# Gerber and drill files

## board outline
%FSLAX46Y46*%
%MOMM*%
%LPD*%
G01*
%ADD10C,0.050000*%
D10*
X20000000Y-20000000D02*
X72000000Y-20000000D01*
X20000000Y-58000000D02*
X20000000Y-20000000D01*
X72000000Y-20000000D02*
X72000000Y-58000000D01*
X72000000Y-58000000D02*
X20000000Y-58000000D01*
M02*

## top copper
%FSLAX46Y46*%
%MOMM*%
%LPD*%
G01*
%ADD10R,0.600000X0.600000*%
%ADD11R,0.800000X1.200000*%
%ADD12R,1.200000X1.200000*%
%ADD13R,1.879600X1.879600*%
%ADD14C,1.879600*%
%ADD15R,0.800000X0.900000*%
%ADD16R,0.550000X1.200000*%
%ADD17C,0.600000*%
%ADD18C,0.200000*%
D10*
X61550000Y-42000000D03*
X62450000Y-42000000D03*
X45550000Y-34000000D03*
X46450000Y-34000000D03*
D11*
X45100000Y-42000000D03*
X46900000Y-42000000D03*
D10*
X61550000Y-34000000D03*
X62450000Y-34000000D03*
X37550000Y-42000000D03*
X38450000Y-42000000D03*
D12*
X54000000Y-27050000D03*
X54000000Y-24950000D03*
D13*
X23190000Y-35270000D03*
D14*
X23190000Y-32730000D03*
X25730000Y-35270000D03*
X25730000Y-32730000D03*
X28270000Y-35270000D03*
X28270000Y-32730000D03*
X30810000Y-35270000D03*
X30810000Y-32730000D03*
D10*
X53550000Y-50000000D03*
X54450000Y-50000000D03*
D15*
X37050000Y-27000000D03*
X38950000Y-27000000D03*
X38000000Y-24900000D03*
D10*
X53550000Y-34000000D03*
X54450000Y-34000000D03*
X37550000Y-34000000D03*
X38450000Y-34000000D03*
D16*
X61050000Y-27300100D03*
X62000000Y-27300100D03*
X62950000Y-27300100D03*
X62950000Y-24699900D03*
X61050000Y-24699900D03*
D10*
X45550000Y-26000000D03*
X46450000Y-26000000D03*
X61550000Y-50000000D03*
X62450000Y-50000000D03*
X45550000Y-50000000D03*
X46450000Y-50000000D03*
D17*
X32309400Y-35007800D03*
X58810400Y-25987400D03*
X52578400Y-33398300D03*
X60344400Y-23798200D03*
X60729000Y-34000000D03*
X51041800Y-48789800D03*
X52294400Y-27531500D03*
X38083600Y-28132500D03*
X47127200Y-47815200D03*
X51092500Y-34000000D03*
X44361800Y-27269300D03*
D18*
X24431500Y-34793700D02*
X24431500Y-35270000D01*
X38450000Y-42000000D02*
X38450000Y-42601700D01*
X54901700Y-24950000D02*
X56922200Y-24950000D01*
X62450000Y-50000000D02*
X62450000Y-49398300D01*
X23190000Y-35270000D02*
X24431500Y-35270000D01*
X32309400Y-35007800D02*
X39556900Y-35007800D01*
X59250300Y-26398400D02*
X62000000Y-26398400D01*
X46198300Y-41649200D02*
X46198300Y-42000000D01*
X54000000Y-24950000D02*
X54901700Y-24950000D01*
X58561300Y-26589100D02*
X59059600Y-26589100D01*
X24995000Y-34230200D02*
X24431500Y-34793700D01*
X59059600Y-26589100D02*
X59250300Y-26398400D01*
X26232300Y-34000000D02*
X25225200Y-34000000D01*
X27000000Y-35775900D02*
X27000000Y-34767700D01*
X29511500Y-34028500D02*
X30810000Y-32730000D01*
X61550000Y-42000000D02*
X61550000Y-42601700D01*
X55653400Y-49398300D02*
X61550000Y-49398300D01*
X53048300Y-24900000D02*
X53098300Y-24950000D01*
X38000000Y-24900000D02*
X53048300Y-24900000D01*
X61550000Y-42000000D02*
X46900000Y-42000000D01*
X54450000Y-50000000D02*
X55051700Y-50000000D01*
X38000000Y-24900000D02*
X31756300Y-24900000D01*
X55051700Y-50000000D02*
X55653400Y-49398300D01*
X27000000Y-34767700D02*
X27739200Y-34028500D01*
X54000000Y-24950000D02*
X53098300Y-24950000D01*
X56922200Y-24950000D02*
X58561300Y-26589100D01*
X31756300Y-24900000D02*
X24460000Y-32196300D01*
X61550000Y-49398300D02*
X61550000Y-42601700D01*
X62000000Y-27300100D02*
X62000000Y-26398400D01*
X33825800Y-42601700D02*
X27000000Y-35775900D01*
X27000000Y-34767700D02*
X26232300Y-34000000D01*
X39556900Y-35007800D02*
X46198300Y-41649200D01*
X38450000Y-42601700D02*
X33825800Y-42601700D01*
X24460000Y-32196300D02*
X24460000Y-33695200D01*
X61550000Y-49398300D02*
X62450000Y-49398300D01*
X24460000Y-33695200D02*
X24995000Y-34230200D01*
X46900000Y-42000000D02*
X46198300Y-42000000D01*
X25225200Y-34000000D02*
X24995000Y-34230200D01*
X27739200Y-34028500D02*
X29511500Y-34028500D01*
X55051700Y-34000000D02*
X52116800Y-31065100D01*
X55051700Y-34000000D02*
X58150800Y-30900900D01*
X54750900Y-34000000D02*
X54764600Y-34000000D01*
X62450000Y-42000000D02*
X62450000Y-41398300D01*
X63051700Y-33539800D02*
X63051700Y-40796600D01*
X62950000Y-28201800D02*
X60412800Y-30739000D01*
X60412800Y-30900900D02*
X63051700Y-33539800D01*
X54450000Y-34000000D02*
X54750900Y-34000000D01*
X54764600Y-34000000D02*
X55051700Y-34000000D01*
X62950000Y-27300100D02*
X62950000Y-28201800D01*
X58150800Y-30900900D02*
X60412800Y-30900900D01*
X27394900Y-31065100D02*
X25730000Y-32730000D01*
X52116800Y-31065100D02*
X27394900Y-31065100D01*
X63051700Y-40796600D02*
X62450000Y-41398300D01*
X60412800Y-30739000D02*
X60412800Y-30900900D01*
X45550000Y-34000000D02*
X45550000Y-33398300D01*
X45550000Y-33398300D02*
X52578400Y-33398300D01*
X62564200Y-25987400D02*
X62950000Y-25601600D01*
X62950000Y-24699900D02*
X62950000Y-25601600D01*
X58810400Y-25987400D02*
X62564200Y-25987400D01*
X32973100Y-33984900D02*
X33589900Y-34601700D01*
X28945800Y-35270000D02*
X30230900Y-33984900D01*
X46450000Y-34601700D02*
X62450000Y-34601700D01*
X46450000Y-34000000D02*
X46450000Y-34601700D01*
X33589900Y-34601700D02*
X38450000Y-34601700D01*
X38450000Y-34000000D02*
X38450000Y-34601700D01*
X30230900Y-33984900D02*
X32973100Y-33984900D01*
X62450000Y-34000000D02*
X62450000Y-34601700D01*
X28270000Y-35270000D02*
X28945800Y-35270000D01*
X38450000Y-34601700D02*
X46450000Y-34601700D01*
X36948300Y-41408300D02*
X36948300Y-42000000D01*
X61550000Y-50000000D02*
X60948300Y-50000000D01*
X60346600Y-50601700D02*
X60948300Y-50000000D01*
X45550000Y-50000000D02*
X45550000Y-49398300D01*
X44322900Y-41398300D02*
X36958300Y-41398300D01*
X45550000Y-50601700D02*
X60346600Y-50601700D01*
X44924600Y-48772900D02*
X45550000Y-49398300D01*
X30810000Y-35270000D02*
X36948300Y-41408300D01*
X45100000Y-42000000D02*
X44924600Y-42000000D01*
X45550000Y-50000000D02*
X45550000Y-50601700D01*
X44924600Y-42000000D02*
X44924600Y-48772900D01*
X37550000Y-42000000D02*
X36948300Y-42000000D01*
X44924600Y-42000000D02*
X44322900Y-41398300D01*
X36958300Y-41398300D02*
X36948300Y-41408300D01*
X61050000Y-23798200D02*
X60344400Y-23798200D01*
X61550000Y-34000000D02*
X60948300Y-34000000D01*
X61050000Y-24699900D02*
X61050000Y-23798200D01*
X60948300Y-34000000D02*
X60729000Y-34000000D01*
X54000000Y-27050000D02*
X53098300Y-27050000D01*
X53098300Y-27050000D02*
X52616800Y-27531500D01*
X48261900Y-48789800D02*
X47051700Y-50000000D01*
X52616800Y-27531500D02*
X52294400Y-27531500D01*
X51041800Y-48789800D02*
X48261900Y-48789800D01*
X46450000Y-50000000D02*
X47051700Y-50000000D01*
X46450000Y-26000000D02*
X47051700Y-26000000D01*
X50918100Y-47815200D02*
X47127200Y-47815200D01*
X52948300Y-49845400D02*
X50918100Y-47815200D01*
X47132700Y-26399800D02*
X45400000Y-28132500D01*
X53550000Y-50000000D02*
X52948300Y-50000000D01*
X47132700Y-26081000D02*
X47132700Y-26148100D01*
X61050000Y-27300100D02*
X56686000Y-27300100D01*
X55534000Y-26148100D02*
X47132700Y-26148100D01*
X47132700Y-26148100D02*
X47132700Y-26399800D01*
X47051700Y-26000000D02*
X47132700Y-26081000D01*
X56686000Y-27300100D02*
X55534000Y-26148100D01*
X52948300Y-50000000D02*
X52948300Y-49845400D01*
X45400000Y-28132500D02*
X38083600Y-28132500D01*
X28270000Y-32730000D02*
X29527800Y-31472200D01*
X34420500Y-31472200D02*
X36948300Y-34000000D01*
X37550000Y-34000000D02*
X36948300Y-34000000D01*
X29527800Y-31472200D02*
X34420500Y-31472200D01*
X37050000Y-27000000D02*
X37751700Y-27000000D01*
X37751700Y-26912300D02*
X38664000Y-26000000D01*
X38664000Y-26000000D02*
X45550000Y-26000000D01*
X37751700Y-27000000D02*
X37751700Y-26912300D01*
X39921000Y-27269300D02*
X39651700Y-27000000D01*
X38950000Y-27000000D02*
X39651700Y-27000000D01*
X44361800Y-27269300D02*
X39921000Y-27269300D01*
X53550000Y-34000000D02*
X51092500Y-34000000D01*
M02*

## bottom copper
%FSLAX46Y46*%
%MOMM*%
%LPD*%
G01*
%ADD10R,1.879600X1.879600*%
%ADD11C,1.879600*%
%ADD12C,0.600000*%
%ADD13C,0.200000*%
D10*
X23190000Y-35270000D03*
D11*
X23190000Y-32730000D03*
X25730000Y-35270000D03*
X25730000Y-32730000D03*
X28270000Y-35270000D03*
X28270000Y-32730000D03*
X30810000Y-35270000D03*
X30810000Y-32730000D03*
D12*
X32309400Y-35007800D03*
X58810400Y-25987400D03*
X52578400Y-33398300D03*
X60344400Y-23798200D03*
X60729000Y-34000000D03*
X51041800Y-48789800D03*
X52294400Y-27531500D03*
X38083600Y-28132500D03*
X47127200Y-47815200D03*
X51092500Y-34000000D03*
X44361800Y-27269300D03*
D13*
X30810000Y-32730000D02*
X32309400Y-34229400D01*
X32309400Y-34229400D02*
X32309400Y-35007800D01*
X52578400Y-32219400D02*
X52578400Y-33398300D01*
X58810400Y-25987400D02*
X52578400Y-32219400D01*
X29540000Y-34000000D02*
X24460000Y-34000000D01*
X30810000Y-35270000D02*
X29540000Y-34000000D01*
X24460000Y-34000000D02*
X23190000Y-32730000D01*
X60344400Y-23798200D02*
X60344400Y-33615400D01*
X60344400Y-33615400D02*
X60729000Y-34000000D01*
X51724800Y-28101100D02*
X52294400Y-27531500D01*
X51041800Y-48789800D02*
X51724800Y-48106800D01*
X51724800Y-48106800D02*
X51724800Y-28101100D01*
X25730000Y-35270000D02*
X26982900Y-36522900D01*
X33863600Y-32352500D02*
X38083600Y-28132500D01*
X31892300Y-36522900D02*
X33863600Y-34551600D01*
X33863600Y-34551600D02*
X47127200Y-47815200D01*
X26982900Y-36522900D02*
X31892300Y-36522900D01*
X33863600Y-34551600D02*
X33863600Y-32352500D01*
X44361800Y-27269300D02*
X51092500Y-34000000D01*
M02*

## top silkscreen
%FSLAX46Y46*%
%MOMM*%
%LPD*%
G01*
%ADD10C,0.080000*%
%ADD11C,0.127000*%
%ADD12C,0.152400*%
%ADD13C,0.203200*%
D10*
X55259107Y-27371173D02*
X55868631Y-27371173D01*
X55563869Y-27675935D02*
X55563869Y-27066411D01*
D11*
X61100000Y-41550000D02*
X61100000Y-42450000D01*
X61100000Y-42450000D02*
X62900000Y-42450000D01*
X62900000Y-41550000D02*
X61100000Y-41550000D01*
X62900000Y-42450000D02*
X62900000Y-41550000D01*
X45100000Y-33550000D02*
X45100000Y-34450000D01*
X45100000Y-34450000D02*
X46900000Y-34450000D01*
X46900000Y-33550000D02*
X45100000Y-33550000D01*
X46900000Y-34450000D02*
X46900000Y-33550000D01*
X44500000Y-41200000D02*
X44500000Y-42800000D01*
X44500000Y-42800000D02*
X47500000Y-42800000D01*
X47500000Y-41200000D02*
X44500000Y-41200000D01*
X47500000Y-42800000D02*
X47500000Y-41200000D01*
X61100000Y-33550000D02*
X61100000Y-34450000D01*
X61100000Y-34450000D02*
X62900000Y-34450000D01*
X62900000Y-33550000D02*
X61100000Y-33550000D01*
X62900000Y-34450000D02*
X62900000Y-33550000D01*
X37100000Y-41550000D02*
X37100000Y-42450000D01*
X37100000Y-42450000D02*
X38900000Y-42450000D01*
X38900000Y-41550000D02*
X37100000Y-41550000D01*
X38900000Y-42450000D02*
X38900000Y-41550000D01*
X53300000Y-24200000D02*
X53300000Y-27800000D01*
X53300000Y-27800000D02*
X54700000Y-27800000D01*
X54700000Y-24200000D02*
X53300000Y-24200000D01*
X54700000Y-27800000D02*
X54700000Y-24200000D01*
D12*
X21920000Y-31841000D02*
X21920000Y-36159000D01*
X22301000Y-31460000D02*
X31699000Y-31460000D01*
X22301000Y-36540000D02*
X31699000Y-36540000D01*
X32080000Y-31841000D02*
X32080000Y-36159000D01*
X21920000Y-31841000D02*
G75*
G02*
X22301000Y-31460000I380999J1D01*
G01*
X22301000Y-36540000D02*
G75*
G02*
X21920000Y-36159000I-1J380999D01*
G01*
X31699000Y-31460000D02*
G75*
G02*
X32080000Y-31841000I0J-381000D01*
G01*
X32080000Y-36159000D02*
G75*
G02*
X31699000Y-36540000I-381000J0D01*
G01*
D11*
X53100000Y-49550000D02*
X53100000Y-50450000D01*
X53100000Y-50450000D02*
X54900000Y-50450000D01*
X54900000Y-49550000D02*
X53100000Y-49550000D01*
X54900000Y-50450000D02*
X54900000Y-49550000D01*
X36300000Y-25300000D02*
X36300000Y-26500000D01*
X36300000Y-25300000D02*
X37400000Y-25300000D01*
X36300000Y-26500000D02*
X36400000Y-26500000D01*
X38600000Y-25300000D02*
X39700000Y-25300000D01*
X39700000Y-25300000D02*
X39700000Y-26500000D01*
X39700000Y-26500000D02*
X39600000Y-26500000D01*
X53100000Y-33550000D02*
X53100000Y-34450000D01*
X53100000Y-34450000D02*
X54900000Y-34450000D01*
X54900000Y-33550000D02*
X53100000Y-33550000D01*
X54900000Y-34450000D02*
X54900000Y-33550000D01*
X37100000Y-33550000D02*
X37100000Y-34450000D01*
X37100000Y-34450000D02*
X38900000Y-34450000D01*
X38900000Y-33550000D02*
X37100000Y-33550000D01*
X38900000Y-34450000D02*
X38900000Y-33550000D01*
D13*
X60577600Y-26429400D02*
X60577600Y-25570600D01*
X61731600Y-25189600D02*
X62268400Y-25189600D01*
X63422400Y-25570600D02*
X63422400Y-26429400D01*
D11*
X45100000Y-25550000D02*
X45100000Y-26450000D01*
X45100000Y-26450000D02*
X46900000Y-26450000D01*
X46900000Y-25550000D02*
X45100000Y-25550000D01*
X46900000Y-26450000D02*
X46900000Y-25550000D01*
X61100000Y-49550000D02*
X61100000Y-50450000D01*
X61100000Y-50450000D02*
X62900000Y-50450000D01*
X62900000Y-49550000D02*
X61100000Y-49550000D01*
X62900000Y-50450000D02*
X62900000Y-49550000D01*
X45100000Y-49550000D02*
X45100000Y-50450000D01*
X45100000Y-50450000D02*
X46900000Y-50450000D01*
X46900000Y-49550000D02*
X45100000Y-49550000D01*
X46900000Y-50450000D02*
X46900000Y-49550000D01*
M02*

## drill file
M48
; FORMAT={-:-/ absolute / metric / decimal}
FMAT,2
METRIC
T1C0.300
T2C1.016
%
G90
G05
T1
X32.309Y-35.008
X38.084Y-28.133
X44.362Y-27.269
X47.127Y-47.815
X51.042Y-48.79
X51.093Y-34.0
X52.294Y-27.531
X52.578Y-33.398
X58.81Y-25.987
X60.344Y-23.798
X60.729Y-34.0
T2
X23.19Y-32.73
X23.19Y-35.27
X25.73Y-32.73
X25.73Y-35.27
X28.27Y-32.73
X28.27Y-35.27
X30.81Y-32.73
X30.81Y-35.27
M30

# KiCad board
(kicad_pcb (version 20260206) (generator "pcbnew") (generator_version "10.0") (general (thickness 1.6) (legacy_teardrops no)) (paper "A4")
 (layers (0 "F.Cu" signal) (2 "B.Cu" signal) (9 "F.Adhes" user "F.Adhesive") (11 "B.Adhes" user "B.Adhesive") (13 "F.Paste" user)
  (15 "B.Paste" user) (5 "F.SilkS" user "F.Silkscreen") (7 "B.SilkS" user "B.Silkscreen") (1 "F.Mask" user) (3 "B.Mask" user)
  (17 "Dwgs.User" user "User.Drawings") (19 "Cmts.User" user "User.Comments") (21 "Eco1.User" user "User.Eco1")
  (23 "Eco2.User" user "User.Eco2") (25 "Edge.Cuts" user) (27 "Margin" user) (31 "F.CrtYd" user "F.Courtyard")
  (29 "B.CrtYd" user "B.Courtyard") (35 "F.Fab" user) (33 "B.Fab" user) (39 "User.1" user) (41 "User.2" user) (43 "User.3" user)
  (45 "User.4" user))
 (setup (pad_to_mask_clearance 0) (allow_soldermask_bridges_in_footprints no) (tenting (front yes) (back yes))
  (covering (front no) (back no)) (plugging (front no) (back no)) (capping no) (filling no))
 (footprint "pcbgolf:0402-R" (layer "F.Cu") (at 62 42)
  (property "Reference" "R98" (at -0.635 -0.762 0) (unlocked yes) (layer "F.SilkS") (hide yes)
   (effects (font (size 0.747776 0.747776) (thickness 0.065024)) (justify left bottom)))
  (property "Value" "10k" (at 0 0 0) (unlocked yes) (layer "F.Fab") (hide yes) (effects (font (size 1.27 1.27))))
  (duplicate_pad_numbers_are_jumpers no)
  (fp_line (start -0.9 -0.45) (end -0.9 0.45) (stroke (width 0.127) (type solid)) (layer "F.SilkS"))
  (fp_line (start -0.9 0.45) (end 0.9 0.45) (stroke (width 0.127) (type solid)) (layer "F.SilkS"))
  (fp_line (start 0.9 -0.45) (end -0.9 -0.45) (stroke (width 0.127) (type solid)) (layer "F.SilkS"))
  (fp_line (start 0.9 0.45) (end 0.9 -0.45) (stroke (width 0.127) (type solid)) (layer "F.SilkS"))
  (pad "1" smd rect (at -0.45 0) (size 0.6 0.6) (layers "F.Cu" "F.Mask" "F.Paste") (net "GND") (solder_mask_margin 0.0508)
   (solder_paste_margin 0) (thermal_bridge_angle 0))
  (pad "2" smd rect (at 0.45 0) (size 0.6 0.6) (layers "F.Cu" "F.Mask" "F.Paste") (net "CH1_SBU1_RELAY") (solder_mask_margin 0.0508)
   (solder_paste_margin 0) (thermal_bridge_angle 0)))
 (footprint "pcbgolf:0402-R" (layer "F.Cu") (at 46 34)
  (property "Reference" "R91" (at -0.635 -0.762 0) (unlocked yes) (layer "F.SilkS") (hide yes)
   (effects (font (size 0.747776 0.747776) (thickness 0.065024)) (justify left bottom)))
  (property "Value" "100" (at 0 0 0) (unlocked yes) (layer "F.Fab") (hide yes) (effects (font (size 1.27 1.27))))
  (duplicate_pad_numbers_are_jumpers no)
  (fp_line (start -0.9 -0.45) (end -0.9 0.45) (stroke (width 0.127) (type solid)) (layer "F.SilkS"))
  (fp_line (start -0.9 0.45) (end 0.9 0.45) (stroke (width 0.127) (type solid)) (layer "F.SilkS"))
  (fp_line (start 0.9 -0.45) (end -0.9 -0.45) (stroke (width 0.127) (type solid)) (layer "F.SilkS"))
  (fp_line (start 0.9 0.45) (end 0.9 -0.45) (stroke (width 0.127) (type solid)) (layer "F.SilkS"))
  (pad "1" smd rect (at -0.45 0) (size 0.6 0.6) (layers "F.Cu" "F.Mask" "F.Paste") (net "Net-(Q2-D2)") (solder_mask_margin 0.0508)
   (solder_paste_margin 0) (thermal_bridge_angle 0))
  (pad "2" smd rect (at 0.45 0) (size 0.6 0.6) (layers "F.Cu" "F.Mask" "F.Paste") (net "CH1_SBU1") (solder_mask_margin 0.0508)
   (solder_paste_margin 0) (thermal_bridge_angle 0)))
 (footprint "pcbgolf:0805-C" (layer "F.Cu") (at 46 42)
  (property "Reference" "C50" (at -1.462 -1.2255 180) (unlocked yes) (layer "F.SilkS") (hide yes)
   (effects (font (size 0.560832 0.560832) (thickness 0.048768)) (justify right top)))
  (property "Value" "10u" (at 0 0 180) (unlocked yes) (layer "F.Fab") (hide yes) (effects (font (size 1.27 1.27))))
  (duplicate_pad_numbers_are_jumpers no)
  (fp_line (start -1.5 -0.8) (end -1.5 0.8) (stroke (width 0.127) (type solid)) (layer "F.SilkS"))
  (fp_line (start -1.5 0.8) (end 1.5 0.8) (stroke (width 0.127) (type solid)) (layer "F.SilkS"))
  (fp_line (start 1.5 -0.8) (end -1.5 -0.8) (stroke (width 0.127) (type solid)) (layer "F.SilkS"))
  (fp_line (start 1.5 0.8) (end 1.5 -0.8) (stroke (width 0.127) (type solid)) (layer "F.SilkS"))
  (pad "1" smd rect (at -0.9 0) (size 0.8 1.2) (layers "F.Cu" "F.Mask" "F.Paste") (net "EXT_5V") (solder_mask_margin 0.0508)
   (solder_paste_margin 0) (thermal_bridge_angle 0))
  (pad "2" smd rect (at 0.9 0) (size 0.8 1.2) (layers "F.Cu" "F.Mask" "F.Paste") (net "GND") (solder_mask_margin 0.0508)
   (solder_paste_margin 0) (thermal_bridge_angle 0)))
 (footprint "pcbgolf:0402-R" (layer "F.Cu") (at 62 34)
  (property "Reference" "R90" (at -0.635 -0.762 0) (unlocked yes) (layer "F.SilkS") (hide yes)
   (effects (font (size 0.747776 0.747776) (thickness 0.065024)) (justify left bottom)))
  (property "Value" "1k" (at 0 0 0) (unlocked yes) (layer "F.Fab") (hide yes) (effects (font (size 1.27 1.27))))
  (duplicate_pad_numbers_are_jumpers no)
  (fp_line (start -0.9 -0.45) (end -0.9 0.45) (stroke (width 0.127) (type solid)) (layer "F.SilkS"))
  (fp_line (start -0.9 0.45) (end 0.9 0.45) (stroke (width 0.127) (type solid)) (layer "F.SilkS"))
  (fp_line (start 0.9 -0.45) (end -0.9 -0.45) (stroke (width 0.127) (type solid)) (layer "F.SilkS"))
  (fp_line (start 0.9 0.45) (end 0.9 -0.45) (stroke (width 0.127) (type solid)) (layer "F.SilkS"))
  (pad "1" smd rect (at -0.45 0) (size 0.6 0.6) (layers "F.Cu" "F.Mask" "F.Paste") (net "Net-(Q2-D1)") (solder_mask_margin 0.0508)
   (solder_paste_margin 0) (thermal_bridge_angle 0))
  (pad "2" smd rect (at 0.45 0) (size 0.6 0.6) (layers "F.Cu" "F.Mask" "F.Paste") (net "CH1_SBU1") (solder_mask_margin 0.0508)
   (solder_paste_margin 0) (thermal_bridge_angle 0)))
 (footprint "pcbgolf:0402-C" (layer "F.Cu") (at 38 42)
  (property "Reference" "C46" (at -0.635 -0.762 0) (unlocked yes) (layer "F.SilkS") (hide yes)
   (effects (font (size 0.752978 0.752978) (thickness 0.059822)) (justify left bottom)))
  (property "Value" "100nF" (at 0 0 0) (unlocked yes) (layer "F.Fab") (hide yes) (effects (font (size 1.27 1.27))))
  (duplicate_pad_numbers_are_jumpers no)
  (fp_line (start -0.9 -0.45) (end -0.9 0.45) (stroke (width 0.127) (type solid)) (layer "F.SilkS"))
  (fp_line (start -0.9 0.45) (end 0.9 0.45) (stroke (width 0.127) (type solid)) (layer "F.SilkS"))
  (fp_line (start 0.9 -0.45) (end -0.9 -0.45) (stroke (width 0.127) (type solid)) (layer "F.SilkS"))
  (fp_line (start 0.9 0.45) (end 0.9 -0.45) (stroke (width 0.127) (type solid)) (layer "F.SilkS"))
  (pad "1" smd rect (at -0.45 0) (size 0.6 0.6) (layers "F.Cu" "F.Mask" "F.Paste") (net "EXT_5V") (solder_mask_margin 0.0508)
   (solder_paste_margin 0) (thermal_bridge_angle 0))
  (pad "2" smd rect (at 0.45 0) (size 0.6 0.6) (layers "F.Cu" "F.Mask" "F.Paste") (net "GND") (solder_mask_margin 0.0508)
   (solder_paste_margin 0) (thermal_bridge_angle 0)))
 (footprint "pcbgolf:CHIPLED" (layer "F.Cu") (at 54 26)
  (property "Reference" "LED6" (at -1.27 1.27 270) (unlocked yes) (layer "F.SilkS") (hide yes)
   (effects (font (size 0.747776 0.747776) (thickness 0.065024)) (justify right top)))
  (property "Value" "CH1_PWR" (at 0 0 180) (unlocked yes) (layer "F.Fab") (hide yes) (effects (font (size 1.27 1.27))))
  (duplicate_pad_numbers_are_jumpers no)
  (fp_line (start -0.7 -1.8) (end -0.7 1.8) (stroke (width 0.127) (type solid)) (layer "F.SilkS"))
  (fp_line (start -0.7 1.8) (end 0.7 1.8) (stroke (width 0.127) (type solid)) (layer "F.SilkS"))
  (fp_line (start 0.7 -1.8) (end -0.7 -1.8) (stroke (width 0.127) (type solid)) (layer "F.SilkS"))
  (fp_line (start 0.7 1.8) (end 0.7 -1.8) (stroke (width 0.127) (type solid)) (layer "F.SilkS"))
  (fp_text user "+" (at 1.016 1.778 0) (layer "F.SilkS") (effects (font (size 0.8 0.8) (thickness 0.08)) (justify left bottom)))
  (pad "A" smd rect (at 0 1.05) (size 1.2 1.2) (layers "F.Cu" "F.Mask" "F.Paste") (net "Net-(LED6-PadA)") (solder_mask_margin 0.0508)
   (solder_paste_margin 0) (thermal_bridge_angle 0))
  (pad "C" smd rect (at 0 -1.05) (size 1.2 1.2) (layers "F.Cu" "F.Mask" "F.Paste") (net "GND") (solder_mask_margin 0.0508)
   (solder_paste_margin 0) (thermal_bridge_angle 0)))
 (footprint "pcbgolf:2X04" (layer "F.Cu") (at 27 34)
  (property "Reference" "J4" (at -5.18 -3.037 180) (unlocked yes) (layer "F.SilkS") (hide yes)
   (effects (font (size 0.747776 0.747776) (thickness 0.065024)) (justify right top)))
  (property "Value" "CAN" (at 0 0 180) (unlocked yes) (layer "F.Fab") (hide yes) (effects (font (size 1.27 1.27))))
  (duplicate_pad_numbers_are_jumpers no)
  (fp_line (start -5.08 -2.159) (end -5.08 2.159) (stroke (width 0.1524) (type solid)) (layer "F.SilkS"))
  (fp_line (start -4.699 -2.54) (end 4.699 -2.54) (stroke (width 0.1524) (type solid)) (layer "F.SilkS"))
  (fp_line (start -4.699 2.54) (end 4.699 2.54) (stroke (width 0.1524) (type solid)) (layer "F.SilkS"))
  (fp_line (start 5.08 -2.159) (end 5.08 2.159) (stroke (width 0.1524) (type solid)) (layer "F.SilkS"))
  (fp_arc (start -5.08 -2.159) (mid -4.968408 -2.428408) (end -4.699 -2.54) (stroke (width 0.1524) (type solid)) (layer "F.SilkS"))
  (fp_arc (start -4.699 2.54) (mid -4.968408 2.428408) (end -5.08 2.159) (stroke (width 0.1524) (type solid)) (layer "F.SilkS"))
  (fp_arc (start 4.699 -2.54) (mid 4.968408 -2.428408) (end 5.08 -2.159) (stroke (width 0.1524) (type solid)) (layer "F.SilkS"))
  (fp_arc (start 5.08 2.159) (mid 4.968408 2.428408) (end 4.699 2.54) (stroke (width 0.1524) (type solid)) (layer "F.SilkS"))
  (pad "1" thru_hole rect (at -3.81 1.27 90) (size 1.8796 1.8796) (drill 1.016) (layers "*.Cu" "*.Mask") (remove_unused_layers no)
   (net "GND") (solder_mask_margin 0.0508) (thermal_bridge_angle 0))
  (pad "2" thru_hole circle (at -3.81 -1.27 90) (size 1.8796 1.8796) (drill 1.016) (layers "*.Cu" "*.Mask") (remove_unused_layers no)
   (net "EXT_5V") (solder_mask_margin 0.0508) (thermal_bridge_angle 0))
  (pad "3" thru_hole circle (at -1.27 1.27 90) (size 1.8796 1.8796) (drill 1.016) (layers "*.Cu" "*.Mask") (remove_unused_layers no)
   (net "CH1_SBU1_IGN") (solder_mask_margin 0.0508) (thermal_bridge_angle 0))
  (pad "4" thru_hole circle (at -1.27 -1.27 90) (size 1.8796 1.8796) (drill 1.016) (layers "*.Cu" "*.Mask") (remove_unused_layers no)
   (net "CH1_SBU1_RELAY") (solder_mask_margin 0.0508) (thermal_bridge_angle 0))
  (pad "5" thru_hole circle (at 1.27 1.27 90) (size 1.8796 1.8796) (drill 1.016) (layers "*.Cu" "*.Mask") (remove_unused_layers no)
   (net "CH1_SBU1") (solder_mask_margin 0.0508) (thermal_bridge_angle 0))
  (pad "6" thru_hole circle (at 1.27 -1.27 90) (size 1.8796 1.8796) (drill 1.016) (layers "*.Cu" "*.Mask") (remove_unused_layers no)
   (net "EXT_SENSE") (solder_mask_margin 0.0508) (thermal_bridge_angle 0))
  (pad "7" thru_hole circle (at 3.81 1.27 90) (size 1.8796 1.8796) (drill 1.016) (layers "*.Cu" "*.Mask") (remove_unused_layers no)
   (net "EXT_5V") (solder_mask_margin 0.0508) (thermal_bridge_angle 0))
  (pad "8" thru_hole circle (at 3.81 -1.27 90) (size 1.8796 1.8796) (drill 1.016) (layers "*.Cu" "*.Mask") (remove_unused_layers no)
   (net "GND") (solder_mask_margin 0.0508) (thermal_bridge_angle 0)))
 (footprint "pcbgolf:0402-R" (layer "F.Cu") (at 54 50)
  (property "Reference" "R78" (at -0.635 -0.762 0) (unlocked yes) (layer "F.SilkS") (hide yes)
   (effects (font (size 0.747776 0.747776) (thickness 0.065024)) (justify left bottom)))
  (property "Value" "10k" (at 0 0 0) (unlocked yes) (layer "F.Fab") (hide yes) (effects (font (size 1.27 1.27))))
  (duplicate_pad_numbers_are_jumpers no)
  (fp_line (start -0.9 -0.45) (end -0.9 0.45) (stroke (width 0.127) (type solid)) (layer "F.SilkS"))
  (fp_line (start -0.9 0.45) (end 0.9 0.45) (stroke (width 0.127) (type solid)) (layer "F.SilkS"))
  (fp_line (start 0.9 -0.45) (end -0.9 -0.45) (stroke (width 0.127) (type solid)) (layer "F.SilkS"))
  (fp_line (start 0.9 0.45) (end 0.9 -0.45) (stroke (width 0.127) (type solid)) (layer "F.SilkS"))
  (pad "1" smd rect (at -0.45 0) (size 0.6 0.6) (layers "F.Cu" "F.Mask" "F.Paste") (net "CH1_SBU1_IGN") (solder_mask_margin 0.0508)
   (solder_paste_margin 0) (thermal_bridge_angle 0))
  (pad "2" smd rect (at 0.45 0) (size 0.6 0.6) (layers "F.Cu" "F.Mask" "F.Paste") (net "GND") (solder_mask_margin 0.0508)
   (solder_paste_margin 0) (thermal_bridge_angle 0)))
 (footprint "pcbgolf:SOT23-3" (layer "F.Cu") (at 38 26)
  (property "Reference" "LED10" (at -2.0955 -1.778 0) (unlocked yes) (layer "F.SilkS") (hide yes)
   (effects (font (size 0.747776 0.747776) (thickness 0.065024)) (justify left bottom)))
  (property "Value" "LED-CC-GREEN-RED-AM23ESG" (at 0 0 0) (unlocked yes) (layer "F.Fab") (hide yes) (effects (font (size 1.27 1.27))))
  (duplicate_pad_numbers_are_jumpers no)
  (fp_line (start -1.7 -0.7) (end -1.7 0.5) (stroke (width 0.127) (type solid)) (layer "F.SilkS"))
  (fp_line (start -1.7 -0.7) (end -0.6 -0.7) (stroke (width 0.127) (type solid)) (layer "F.SilkS"))
  (fp_line (start -1.7 0.5) (end -1.6 0.5) (stroke (width 0.127) (type solid)) (layer "F.SilkS"))
  (fp_line (start 0.6 -0.7) (end 1.7 -0.7) (stroke (width 0.127) (type solid)) (layer "F.SilkS"))
  (fp_line (start 1.7 -0.7) (end 1.7 0.5) (stroke (width 0.127) (type solid)) (layer "F.SilkS"))
  (fp_line (start 1.7 0.5) (end 1.6 0.5) (stroke (width 0.127) (type solid)) (layer "F.SilkS"))
  (pad "1" smd rect (at -0.95 1) (size 0.8 0.9) (layers "F.Cu" "F.Mask" "F.Paste") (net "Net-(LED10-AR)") (solder_mask_margin 0.0508)
   (solder_paste_margin 0) (thermal_bridge_angle 0))
  (pad "2" smd rect (at 0.95 1) (size 0.8 0.9) (layers "F.Cu" "F.Mask" "F.Paste") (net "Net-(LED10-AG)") (solder_mask_margin 0.0508)
   (solder_paste_margin 0) (thermal_bridge_angle 0))
  (pad "3" smd rect (at 0 -1.1) (size 0.8 0.9) (layers "F.Cu" "F.Mask" "F.Paste") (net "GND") (solder_mask_margin 0.0508)
   (solder_paste_margin 0) (thermal_bridge_angle 0)))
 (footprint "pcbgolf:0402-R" (layer "F.Cu") (at 54 34)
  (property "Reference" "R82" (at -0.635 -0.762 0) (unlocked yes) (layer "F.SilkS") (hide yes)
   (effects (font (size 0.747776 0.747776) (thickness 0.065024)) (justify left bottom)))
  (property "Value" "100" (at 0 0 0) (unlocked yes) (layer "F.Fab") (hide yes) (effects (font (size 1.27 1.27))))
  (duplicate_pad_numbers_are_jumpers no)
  (fp_line (start -0.9 -0.45) (end -0.9 0.45) (stroke (width 0.127) (type solid)) (layer "F.SilkS"))
  (fp_line (start -0.9 0.45) (end 0.9 0.45) (stroke (width 0.127) (type solid)) (layer "F.SilkS"))
  (fp_line (start 0.9 -0.45) (end -0.9 -0.45) (stroke (width 0.127) (type solid)) (layer "F.SilkS"))
  (fp_line (start 0.9 0.45) (end 0.9 -0.45) (stroke (width 0.127) (type solid)) (layer "F.SilkS"))
  (pad "1" smd rect (at -0.45 0) (size 0.6 0.6) (layers "F.Cu" "F.Mask" "F.Paste") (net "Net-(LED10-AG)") (solder_mask_margin 0.0508)
   (solder_paste_margin 0) (thermal_bridge_angle 0))
  (pad "2" smd rect (at 0.45 0) (size 0.6 0.6) (layers "F.Cu" "F.Mask" "F.Paste") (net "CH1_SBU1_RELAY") (solder_mask_margin 0.0508)
   (solder_paste_margin 0) (thermal_bridge_angle 0)))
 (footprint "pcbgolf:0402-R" (layer "F.Cu") (at 38 34)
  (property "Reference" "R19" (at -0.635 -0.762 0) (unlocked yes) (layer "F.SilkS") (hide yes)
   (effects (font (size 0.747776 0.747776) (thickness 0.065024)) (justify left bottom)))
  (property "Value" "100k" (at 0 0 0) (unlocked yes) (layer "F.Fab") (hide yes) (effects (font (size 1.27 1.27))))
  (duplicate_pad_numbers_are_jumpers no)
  (fp_line (start -0.9 -0.45) (end -0.9 0.45) (stroke (width 0.127) (type solid)) (layer "F.SilkS"))
  (fp_line (start -0.9 0.45) (end 0.9 0.45) (stroke (width 0.127) (type solid)) (layer "F.SilkS"))
  (fp_line (start 0.9 -0.45) (end -0.9 -0.45) (stroke (width 0.127) (type solid)) (layer "F.SilkS"))
  (fp_line (start 0.9 0.45) (end 0.9 -0.45) (stroke (width 0.127) (type solid)) (layer "F.SilkS"))
  (pad "1" smd rect (at -0.45 0) (size 0.6 0.6) (layers "F.Cu" "F.Mask" "F.Paste") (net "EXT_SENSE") (solder_mask_margin 0.0508)
   (solder_paste_margin 0) (thermal_bridge_angle 0))
  (pad "2" smd rect (at 0.45 0) (size 0.6 0.6) (layers "F.Cu" "F.Mask" "F.Paste") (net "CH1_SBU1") (solder_mask_margin 0.0508)
   (solder_paste_margin 0) (thermal_bridge_angle 0)))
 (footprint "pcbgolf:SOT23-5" (layer "F.Cu") (at 62 26)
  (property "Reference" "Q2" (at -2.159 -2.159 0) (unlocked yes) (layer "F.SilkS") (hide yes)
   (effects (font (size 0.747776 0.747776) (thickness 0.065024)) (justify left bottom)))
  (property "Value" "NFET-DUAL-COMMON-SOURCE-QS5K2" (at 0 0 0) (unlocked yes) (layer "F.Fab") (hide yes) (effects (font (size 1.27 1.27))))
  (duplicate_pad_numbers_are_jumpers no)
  (fp_line (start -1.4224 0.4294) (end -1.4224 -0.4294) (stroke (width 0.2032) (type solid)) (layer "F.SilkS"))
  (fp_line (start -0.2684 -0.8104) (end 0.2684 -0.8104) (stroke (width 0.2032) (type solid)) (layer "F.SilkS"))
  (fp_line (start 1.4224 -0.4294) (end 1.4224 0.4294) (stroke (width 0.2032) (type solid)) (layer "F.SilkS"))
  (pad "1" smd rect (at -0.95 1.3001) (size 0.55 1.2) (layers "F.Cu" "F.Mask" "F.Paste") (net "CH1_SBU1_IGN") (solder_mask_margin 0.0508)
   (solder_paste_margin 0) (thermal_bridge_angle 0))
  (pad "2" smd rect (at 0 1.3001) (size 0.55 1.2) (layers "F.Cu" "F.Mask" "F.Paste") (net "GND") (solder_mask_margin 0.0508)
   (solder_paste_margin 0) (thermal_bridge_angle 0))
  (pad "3" smd rect (at 0.95 1.3001) (size 0.55 1.2) (layers "F.Cu" "F.Mask" "F.Paste") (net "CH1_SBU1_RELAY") (solder_mask_margin 0.0508)
   (solder_paste_margin 0) (thermal_bridge_angle 0))
  (pad "4" smd rect (at 0.95 -1.3001) (size 0.55 1.2) (layers "F.Cu" "F.Mask" "F.Paste") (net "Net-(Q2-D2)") (solder_mask_margin 0.0508)
   (solder_paste_margin 0) (thermal_bridge_angle 0))
  (pad "5" smd rect (at -0.95 -1.3001) (size 0.55 1.2) (layers "F.Cu" "F.Mask" "F.Paste") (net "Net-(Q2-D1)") (solder_mask_margin 0.0508)
   (solder_paste_margin 0) (thermal_bridge_angle 0)))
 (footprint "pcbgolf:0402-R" (layer "F.Cu") (at 46 26)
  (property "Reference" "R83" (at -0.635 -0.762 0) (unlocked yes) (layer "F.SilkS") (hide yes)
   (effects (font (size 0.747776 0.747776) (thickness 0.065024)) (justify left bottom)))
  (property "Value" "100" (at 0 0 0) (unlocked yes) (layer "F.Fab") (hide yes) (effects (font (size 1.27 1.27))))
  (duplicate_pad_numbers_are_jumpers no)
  (fp_line (start -0.9 -0.45) (end -0.9 0.45) (stroke (width 0.127) (type solid)) (layer "F.SilkS"))
  (fp_line (start -0.9 0.45) (end 0.9 0.45) (stroke (width 0.127) (type solid)) (layer "F.SilkS"))
  (fp_line (start 0.9 -0.45) (end -0.9 -0.45) (stroke (width 0.127) (type solid)) (layer "F.SilkS"))
  (fp_line (start 0.9 0.45) (end 0.9 -0.45) (stroke (width 0.127) (type solid)) (layer "F.SilkS"))
  (pad "1" smd rect (at -0.45 0) (size 0.6 0.6) (layers "F.Cu" "F.Mask" "F.Paste") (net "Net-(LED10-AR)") (solder_mask_margin 0.0508)
   (solder_paste_margin 0) (thermal_bridge_angle 0))
  (pad "2" smd rect (at 0.45 0) (size 0.6 0.6) (layers "F.Cu" "F.Mask" "F.Paste") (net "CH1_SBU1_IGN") (solder_mask_margin 0.0508)
   (solder_paste_margin 0) (thermal_bridge_angle 0)))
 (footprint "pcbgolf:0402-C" (layer "F.Cu") (at 62 50)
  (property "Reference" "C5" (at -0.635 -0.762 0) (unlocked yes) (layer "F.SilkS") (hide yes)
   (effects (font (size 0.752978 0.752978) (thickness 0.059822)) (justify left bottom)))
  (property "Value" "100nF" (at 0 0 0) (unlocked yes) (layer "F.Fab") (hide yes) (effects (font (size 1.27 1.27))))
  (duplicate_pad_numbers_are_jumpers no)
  (fp_line (start -0.9 -0.45) (end -0.9 0.45) (stroke (width 0.127) (type solid)) (layer "F.SilkS"))
  (fp_line (start -0.9 0.45) (end 0.9 0.45) (stroke (width 0.127) (type solid)) (layer "F.SilkS"))
  (fp_line (start 0.9 -0.45) (end -0.9 -0.45) (stroke (width 0.127) (type solid)) (layer "F.SilkS"))
  (fp_line (start 0.9 0.45) (end 0.9 -0.45) (stroke (width 0.127) (type solid)) (layer "F.SilkS"))
  (pad "1" smd rect (at -0.45 0) (size 0.6 0.6) (layers "F.Cu" "F.Mask" "F.Paste") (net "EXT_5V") (solder_mask_margin 0.0508)
   (solder_paste_margin 0) (thermal_bridge_angle 0))
  (pad "2" smd rect (at 0.45 0) (size 0.6 0.6) (layers "F.Cu" "F.Mask" "F.Paste") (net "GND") (solder_mask_margin 0.0508)
   (solder_paste_margin 0) (thermal_bridge_angle 0)))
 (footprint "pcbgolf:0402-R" (layer "F.Cu") (at 46 50)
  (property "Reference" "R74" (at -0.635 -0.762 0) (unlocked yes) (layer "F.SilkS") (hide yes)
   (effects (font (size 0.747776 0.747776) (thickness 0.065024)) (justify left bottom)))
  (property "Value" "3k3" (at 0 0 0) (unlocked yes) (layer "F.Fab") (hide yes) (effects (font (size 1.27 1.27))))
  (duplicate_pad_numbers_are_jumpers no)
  (fp_line (start -0.9 -0.45) (end -0.9 0.45) (stroke (width 0.127) (type solid)) (layer "F.SilkS"))
  (fp_line (start -0.9 0.45) (end 0.9 0.45) (stroke (width 0.127) (type solid)) (layer "F.SilkS"))
  (fp_line (start 0.9 -0.45) (end -0.9 -0.45) (stroke (width 0.127) (type solid)) (layer "F.SilkS"))
  (fp_line (start 0.9 0.45) (end 0.9 -0.45) (stroke (width 0.127) (type solid)) (layer "F.SilkS"))
  (pad "1" smd rect (at -0.45 0) (size 0.6 0.6) (layers "F.Cu" "F.Mask" "F.Paste") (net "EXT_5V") (solder_mask_margin 0.0508)
   (solder_paste_margin 0) (thermal_bridge_angle 0))
  (pad "2" smd rect (at 0.45 0) (size 0.6 0.6) (layers "F.Cu" "F.Mask" "F.Paste") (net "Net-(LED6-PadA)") (solder_mask_margin 0.0508)
   (solder_paste_margin 0) (thermal_bridge_angle 0)))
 (gr_line (start 20 20) (end 72 20) (stroke (width 0.05) (type default)) (layer "Edge.Cuts"))
 (gr_line (start 20 58) (end 20 20) (stroke (width 0.05) (type default)) (layer "Edge.Cuts"))
 (gr_line (start 72 20) (end 72 58) (stroke (width 0.05) (type default)) (layer "Edge.Cuts"))
 (gr_line (start 72 58) (end 20 58) (stroke (width 0.05) (type default)) (layer "Edge.Cuts"))
 (segment (start 24.4315 34.7937) (end 24.4315 35.27) (width 0.2) (layer "F.Cu") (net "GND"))
 (segment (start 38.45 42) (end 38.45 42.6017) (width 0.2) (layer "F.Cu") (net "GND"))
 (segment (start 54.9017 24.95) (end 56.9222 24.95) (width 0.2) (layer "F.Cu") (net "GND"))
 (segment (start 62.45 50) (end 62.45 49.3983) (width 0.2) (layer "F.Cu") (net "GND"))
 (segment (start 23.19 35.27) (end 24.4315 35.27) (width 0.2) (layer "F.Cu") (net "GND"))
 (segment (start 32.3094 35.0078) (end 39.5569 35.0078) (width 0.2) (layer "F.Cu") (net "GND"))
 (segment (start 59.2503 26.3984) (end 62 26.3984) (width 0.2) (layer "F.Cu") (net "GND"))
 (segment (start 46.1983 41.6492) (end 46.1983 42) (width 0.2) (layer "F.Cu") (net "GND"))
 (segment (start 54 24.95) (end 54.9017 24.95) (width 0.2) (layer "F.Cu") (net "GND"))
 (segment (start 58.5613 26.5891) (end 59.0596 26.5891) (width 0.2) (layer "F.Cu") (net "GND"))
 (segment (start 24.995 34.2302) (end 24.4315 34.7937) (width 0.2) (layer "F.Cu") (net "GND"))
 (segment (start 59.0596 26.5891) (end 59.2503 26.3984) (width 0.2) (layer "F.Cu") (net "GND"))
 (segment (start 26.2323 34) (end 25.2252 34) (width 0.2) (layer "F.Cu") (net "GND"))
 (segment (start 27 35.7759) (end 27 34.7677) (width 0.2) (layer "F.Cu") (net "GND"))
 (segment (start 29.5115 34.0285) (end 30.81 32.73) (width 0.2) (layer "F.Cu") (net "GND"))
 (segment (start 61.55 42) (end 61.55 42.6017) (width 0.2) (layer "F.Cu") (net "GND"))
 (segment (start 55.6534 49.3983) (end 61.55 49.3983) (width 0.2) (layer "F.Cu") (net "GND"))
 (segment (start 53.0483 24.9) (end 53.0983 24.95) (width 0.2) (layer "F.Cu") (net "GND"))
 (segment (start 38 24.9) (end 53.0483 24.9) (width 0.2) (layer "F.Cu") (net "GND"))
 (segment (start 61.55 42) (end 46.9 42) (width 0.2) (layer "F.Cu") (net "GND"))
 (segment (start 54.45 50) (end 55.0517 50) (width 0.2) (layer "F.Cu") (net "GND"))
 (segment (start 38 24.9) (end 31.7563 24.9) (width 0.2) (layer "F.Cu") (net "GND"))
 (segment (start 55.0517 50) (end 55.6534 49.3983) (width 0.2) (layer "F.Cu") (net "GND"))
 (segment (start 27 34.7677) (end 27.7392 34.0285) (width 0.2) (layer "F.Cu") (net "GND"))
 (segment (start 54 24.95) (end 53.0983 24.95) (width 0.2) (layer "F.Cu") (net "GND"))
 (segment (start 56.9222 24.95) (end 58.5613 26.5891) (width 0.2) (layer "F.Cu") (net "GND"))
 (segment (start 31.7563 24.9) (end 24.46 32.1963) (width 0.2) (layer "F.Cu") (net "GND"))
 (segment (start 61.55 49.3983) (end 61.55 42.6017) (width 0.2) (layer "F.Cu") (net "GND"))
 (segment (start 62 27.3001) (end 62 26.3984) (width 0.2) (layer "F.Cu") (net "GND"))
 (segment (start 33.8258 42.6017) (end 27 35.7759) (width 0.2) (layer "F.Cu") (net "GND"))
 (segment (start 27 34.7677) (end 26.2323 34) (width 0.2) (layer "F.Cu") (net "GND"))
 (segment (start 39.5569 35.0078) (end 46.1983 41.6492) (width 0.2) (layer "F.Cu") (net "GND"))
 (segment (start 38.45 42.6017) (end 33.8258 42.6017) (width 0.2) (layer "F.Cu") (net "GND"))
 (segment (start 24.46 32.1963) (end 24.46 33.6952) (width 0.2) (layer "F.Cu") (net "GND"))
 (segment (start 61.55 49.3983) (end 62.45 49.3983) (width 0.2) (layer "F.Cu") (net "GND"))
 (segment (start 24.46 33.6952) (end 24.995 34.2302) (width 0.2) (layer "F.Cu") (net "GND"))
 (segment (start 46.9 42) (end 46.1983 42) (width 0.2) (layer "F.Cu") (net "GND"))
 (segment (start 25.2252 34) (end 24.995 34.2302) (width 0.2) (layer "F.Cu") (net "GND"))
 (segment (start 27.7392 34.0285) (end 29.5115 34.0285) (width 0.2) (layer "F.Cu") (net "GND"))
 (via (at 32.3094 35.0078) (size 0.6) (drill 0.3) (layers "F.Cu" "B.Cu") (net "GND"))
 (segment (start 30.81 32.73) (end 32.3094 34.2294) (width 0.2) (layer "B.Cu") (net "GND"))
 (segment (start 32.3094 34.2294) (end 32.3094 35.0078) (width 0.2) (layer "B.Cu") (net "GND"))
 (segment (start 55.0517 34) (end 52.1168 31.0651) (width 0.2) (layer "F.Cu") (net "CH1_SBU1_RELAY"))
 (segment (start 55.0517 34) (end 58.1508 30.9009) (width 0.2) (layer "F.Cu") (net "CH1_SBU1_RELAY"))
 (segment (start 54.7509 34) (end 54.7646 34) (width 0.2) (layer "F.Cu") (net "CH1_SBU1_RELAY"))
 (segment (start 62.45 42) (end 62.45 41.3983) (width 0.2) (layer "F.Cu") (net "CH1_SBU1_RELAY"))
 (segment (start 63.0517 33.5398) (end 63.0517 40.7966) (width 0.2) (layer "F.Cu") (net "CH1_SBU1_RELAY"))
 (segment (start 62.95 28.2018) (end 60.4128 30.739) (width 0.2) (layer "F.Cu") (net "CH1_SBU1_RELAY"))
 (segment (start 60.4128 30.9009) (end 63.0517 33.5398) (width 0.2) (layer "F.Cu") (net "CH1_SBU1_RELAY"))
 (segment (start 54.45 34) (end 54.7509 34) (width 0.2) (layer "F.Cu") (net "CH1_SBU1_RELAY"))
 (segment (start 54.7646 34) (end 55.0517 34) (width 0.2) (layer "F.Cu") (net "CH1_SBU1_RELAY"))
 (segment (start 62.95 27.3001) (end 62.95 28.2018) (width 0.2) (layer "F.Cu") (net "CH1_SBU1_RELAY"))
 (segment (start 58.1508 30.9009) (end 60.4128 30.9009) (width 0.2) (layer "F.Cu") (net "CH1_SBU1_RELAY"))
 (segment (start 27.3949 31.0651) (end 25.73 32.73) (width 0.2) (layer "F.Cu") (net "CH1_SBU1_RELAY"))
 (segment (start 52.1168 31.0651) (end 27.3949 31.0651) (width 0.2) (layer "F.Cu") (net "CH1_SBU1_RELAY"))
 (segment (start 63.0517 40.7966) (end 62.45 41.3983) (width 0.2) (layer "F.Cu") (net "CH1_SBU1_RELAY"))
 (segment (start 60.4128 30.739) (end 60.4128 30.9009) (width 0.2) (layer "F.Cu") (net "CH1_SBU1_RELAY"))
 (segment (start 45.55 34) (end 45.55 33.3983) (width 0.2) (layer "F.Cu") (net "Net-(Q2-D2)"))
 (segment (start 45.55 33.3983) (end 52.5784 33.3983) (width 0.2) (layer "F.Cu") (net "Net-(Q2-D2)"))
 (segment (start 62.5642 25.9874) (end 62.95 25.6016) (width 0.2) (layer "F.Cu") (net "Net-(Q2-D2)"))
 (segment (start 62.95 24.6999) (end 62.95 25.6016) (width 0.2) (layer "F.Cu") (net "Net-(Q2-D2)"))
 (segment (start 58.8104 25.9874) (end 62.5642 25.9874) (width 0.2) (layer "F.Cu") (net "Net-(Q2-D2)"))
 (via (at 58.8104 25.9874) (size 0.6) (drill 0.3) (layers "F.Cu" "B.Cu") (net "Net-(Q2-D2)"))
 (via (at 52.5784 33.3983) (size 0.6) (drill 0.3) (layers "F.Cu" "B.Cu") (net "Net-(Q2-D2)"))
 (segment (start 52.5784 32.2194) (end 52.5784 33.3983) (width 0.2) (layer "B.Cu") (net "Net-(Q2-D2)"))
 (segment (start 58.8104 25.9874) (end 52.5784 32.2194) (width 0.2) (layer "B.Cu") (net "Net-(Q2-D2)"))
 (segment (start 32.9731 33.9849) (end 33.5899 34.6017) (width 0.2) (layer "F.Cu") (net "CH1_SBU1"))
 (segment (start 28.9458 35.27) (end 30.2309 33.9849) (width 0.2) (layer "F.Cu") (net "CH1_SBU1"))
 (segment (start 46.45 34.6017) (end 62.45 34.6017) (width 0.2) (layer "F.Cu") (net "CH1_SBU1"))
 (segment (start 46.45 34) (end 46.45 34.6017) (width 0.2) (layer "F.Cu") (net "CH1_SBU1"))
 (segment (start 33.5899 34.6017) (end 38.45 34.6017) (width 0.2) (layer "F.Cu") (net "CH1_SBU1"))
 (segment (start 38.45 34) (end 38.45 34.6017) (width 0.2) (layer "F.Cu") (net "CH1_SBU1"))
 (segment (start 30.2309 33.9849) (end 32.9731 33.9849) (width 0.2) (layer "F.Cu") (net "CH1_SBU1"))
 (segment (start 62.45 34) (end 62.45 34.6017) (width 0.2) (layer "F.Cu") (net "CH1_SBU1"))
 (segment (start 28.27 35.27) (end 28.9458 35.27) (width 0.2) (layer "F.Cu") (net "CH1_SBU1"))
 (segment (start 38.45 34.6017) (end 46.45 34.6017) (width 0.2) (layer "F.Cu") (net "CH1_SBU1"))
 (segment (start 36.9483 41.4083) (end 36.9483 42) (width 0.2) (layer "F.Cu") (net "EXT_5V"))
 (segment (start 61.55 50) (end 60.9483 50) (width 0.2) (layer "F.Cu") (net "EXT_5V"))
 (segment (start 60.3466 50.6017) (end 60.9483 50) (width 0.2) (layer "F.Cu") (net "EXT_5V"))
 (segment (start 45.55 50) (end 45.55 49.3983) (width 0.2) (layer "F.Cu") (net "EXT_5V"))
 (segment (start 44.3229 41.3983) (end 36.9583 41.3983) (width 0.2) (layer "F.Cu") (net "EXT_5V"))
 (segment (start 45.55 50.6017) (end 60.3466 50.6017) (width 0.2) (layer "F.Cu") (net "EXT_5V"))
 (segment (start 44.9246 48.7729) (end 45.55 49.3983) (width 0.2) (layer "F.Cu") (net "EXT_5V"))
 (segment (start 30.81 35.27) (end 36.9483 41.4083) (width 0.2) (layer "F.Cu") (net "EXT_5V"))
 (segment (start 45.1 42) (end 44.9246 42) (width 0.2) (layer "F.Cu") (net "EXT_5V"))
 (segment (start 45.55 50) (end 45.55 50.6017) (width 0.2) (layer "F.Cu") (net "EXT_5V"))
 (segment (start 44.9246 42) (end 44.9246 48.7729) (width 0.2) (layer "F.Cu") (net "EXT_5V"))
 (segment (start 37.55 42) (end 36.9483 42) (width 0.2) (layer "F.Cu") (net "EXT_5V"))
 (segment (start 44.9246 42) (end 44.3229 41.3983) (width 0.2) (layer "F.Cu") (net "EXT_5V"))
 (segment (start 36.9583 41.3983) (end 36.9483 41.4083) (width 0.2) (layer "F.Cu") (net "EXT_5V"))
 (segment (start 29.54 34) (end 24.46 34) (width 0.2) (layer "B.Cu") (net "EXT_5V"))
 (segment (start 30.81 35.27) (end 29.54 34) (width 0.2) (layer "B.Cu") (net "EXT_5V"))
 (segment (start 24.46 34) (end 23.19 32.73) (width 0.2) (layer "B.Cu") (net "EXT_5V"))
 (segment (start 61.05 23.7982) (end 60.3444 23.7982) (width 0.2) (layer "F.Cu") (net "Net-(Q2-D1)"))
 (segment (start 61.55 34) (end 60.9483 34) (width 0.2) (layer "F.Cu") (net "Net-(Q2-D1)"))
 (segment (start 61.05 24.6999) (end 61.05 23.7982) (width 0.2) (layer "F.Cu") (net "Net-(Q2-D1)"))
 (segment (start 60.9483 34) (end 60.729 34) (width 0.2) (layer "F.Cu") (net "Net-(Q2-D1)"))
 (via (at 60.3444 23.7982) (size 0.6) (drill 0.3) (layers "F.Cu" "B.Cu") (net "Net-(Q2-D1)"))
 (via (at 60.729 34) (size 0.6) (drill 0.3) (layers "F.Cu" "B.Cu") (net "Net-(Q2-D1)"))
 (segment (start 60.3444 23.7982) (end 60.3444 33.6154) (width 0.2) (layer "B.Cu") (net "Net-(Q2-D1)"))
 (segment (start 60.3444 33.6154) (end 60.729 34) (width 0.2) (layer "B.Cu") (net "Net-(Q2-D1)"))
 (segment (start 54 27.05) (end 53.0983 27.05) (width 0.2) (layer "F.Cu") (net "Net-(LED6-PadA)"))
 (segment (start 53.0983 27.05) (end 52.6168 27.5315) (width 0.2) (layer "F.Cu") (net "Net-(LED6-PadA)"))
 (segment (start 48.2619 48.7898) (end 47.0517 50) (width 0.2) (layer "F.Cu") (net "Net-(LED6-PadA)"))
 (segment (start 52.6168 27.5315) (end 52.2944 27.5315) (width 0.2) (layer "F.Cu") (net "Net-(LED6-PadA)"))
 (segment (start 51.0418 48.7898) (end 48.2619 48.7898) (width 0.2) (layer "F.Cu") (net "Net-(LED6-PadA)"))
 (segment (start 46.45 50) (end 47.0517 50) (width 0.2) (layer "F.Cu") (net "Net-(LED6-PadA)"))
 (via (at 51.0418 48.7898) (size 0.6) (drill 0.3) (layers "F.Cu" "B.Cu") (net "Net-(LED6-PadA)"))
 (via (at 52.2944 27.5315) (size 0.6) (drill 0.3) (layers "F.Cu" "B.Cu") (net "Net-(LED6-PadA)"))
 (segment (start 51.7248 28.1011) (end 52.2944 27.5315) (width 0.2) (layer "B.Cu") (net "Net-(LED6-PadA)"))
 (segment (start 51.0418 48.7898) (end 51.7248 48.1068) (width 0.2) (layer "B.Cu") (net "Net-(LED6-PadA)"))
 (segment (start 51.7248 48.1068) (end 51.7248 28.1011) (width 0.2) (layer "B.Cu") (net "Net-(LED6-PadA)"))
 (segment (start 46.45 26) (end 47.0517 26) (width 0.2) (layer "F.Cu") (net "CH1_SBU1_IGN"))
 (segment (start 50.9181 47.8152) (end 47.1272 47.8152) (width 0.2) (layer "F.Cu") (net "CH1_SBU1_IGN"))
 (segment (start 52.9483 49.8454) (end 50.9181 47.8152) (width 0.2) (layer "F.Cu") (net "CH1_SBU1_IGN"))
 (segment (start 47.1327 26.3998) (end 45.4 28.1325) (width 0.2) (layer "F.Cu") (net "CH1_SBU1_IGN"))
 (segment (start 53.55 50) (end 52.9483 50) (width 0.2) (layer "F.Cu") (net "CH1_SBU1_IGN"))
 (segment (start 47.1327 26.081) (end 47.1327 26.1481) (width 0.2) (layer "F.Cu") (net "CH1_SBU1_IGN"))
 (segment (start 61.05 27.3001) (end 56.686 27.3001) (width 0.2) (layer "F.Cu") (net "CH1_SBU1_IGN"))
 (segment (start 55.534 26.1481) (end 47.1327 26.1481) (width 0.2) (layer "F.Cu") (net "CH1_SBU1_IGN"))
 (segment (start 47.1327 26.1481) (end 47.1327 26.3998) (width 0.2) (layer "F.Cu") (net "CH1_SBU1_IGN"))
 (segment (start 47.0517 26) (end 47.1327 26.081) (width 0.2) (layer "F.Cu") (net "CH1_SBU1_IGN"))
 (segment (start 56.686 27.3001) (end 55.534 26.1481) (width 0.2) (layer "F.Cu") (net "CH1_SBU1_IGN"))
 (segment (start 52.9483 50) (end 52.9483 49.8454) (width 0.2) (layer "F.Cu") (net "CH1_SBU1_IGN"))
 (segment (start 45.4 28.1325) (end 38.0836 28.1325) (width 0.2) (layer "F.Cu") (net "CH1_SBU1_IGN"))
 (via (at 38.0836 28.1325) (size 0.6) (drill 0.3) (layers "F.Cu" "B.Cu") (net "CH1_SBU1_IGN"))
 (via (at 47.1272 47.8152) (size 0.6) (drill 0.3) (layers "F.Cu" "B.Cu") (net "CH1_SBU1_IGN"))
 (segment (start 25.73 35.27) (end 26.9829 36.5229) (width 0.2) (layer "B.Cu") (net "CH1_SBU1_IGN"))
 (segment (start 33.8636 32.3525) (end 38.0836 28.1325) (width 0.2) (layer "B.Cu") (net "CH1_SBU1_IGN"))
 (segment (start 31.8923 36.5229) (end 33.8636 34.5516) (width 0.2) (layer "B.Cu") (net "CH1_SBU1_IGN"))
 (segment (start 33.8636 34.5516) (end 47.1272 47.8152) (width 0.2) (layer "B.Cu") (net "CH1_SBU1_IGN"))
 (segment (start 26.9829 36.5229) (end 31.8923 36.5229) (width 0.2) (layer "B.Cu") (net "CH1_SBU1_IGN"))
 (segment (start 33.8636 34.5516) (end 33.8636 32.3525) (width 0.2) (layer "B.Cu") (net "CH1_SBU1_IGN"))
 (segment (start 28.27 32.73) (end 29.5278 31.4722) (width 0.2) (layer "F.Cu") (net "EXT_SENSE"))
 (segment (start 34.4205 31.4722) (end 36.9483 34) (width 0.2) (layer "F.Cu") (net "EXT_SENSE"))
 (segment (start 37.55 34) (end 36.9483 34) (width 0.2) (layer "F.Cu") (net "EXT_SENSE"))
 (segment (start 29.5278 31.4722) (end 34.4205 31.4722) (width 0.2) (layer "F.Cu") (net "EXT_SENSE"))
 (segment (start 37.05 27) (end 37.7517 27) (width 0.2) (layer "F.Cu") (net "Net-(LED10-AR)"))
 (segment (start 37.7517 26.9123) (end 38.664 26) (width 0.2) (layer "F.Cu") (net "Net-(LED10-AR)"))
 (segment (start 38.664 26) (end 45.55 26) (width 0.2) (layer "F.Cu") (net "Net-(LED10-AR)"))
 (segment (start 37.7517 27) (end 37.7517 26.9123) (width 0.2) (layer "F.Cu") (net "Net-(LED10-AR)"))
 (segment (start 39.921 27.2693) (end 39.6517 27) (width 0.2) (layer "F.Cu") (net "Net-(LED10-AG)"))
 (segment (start 38.95 27) (end 39.6517 27) (width 0.2) (layer "F.Cu") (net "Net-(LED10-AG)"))
 (segment (start 44.3618 27.2693) (end 39.921 27.2693) (width 0.2) (layer "F.Cu") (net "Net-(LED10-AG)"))
 (segment (start 53.55 34) (end 51.0925 34) (width 0.2) (layer "F.Cu") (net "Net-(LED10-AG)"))
 (via (at 51.0925 34) (size 0.6) (drill 0.3) (layers "F.Cu" "B.Cu") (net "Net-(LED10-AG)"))
 (via (at 44.3618 27.2693) (size 0.6) (drill 0.3) (layers "F.Cu" "B.Cu") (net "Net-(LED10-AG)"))
 (segment (start 44.3618 27.2693) (end 51.0925 34) (width 0.2) (layer "B.Cu") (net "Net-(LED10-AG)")))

